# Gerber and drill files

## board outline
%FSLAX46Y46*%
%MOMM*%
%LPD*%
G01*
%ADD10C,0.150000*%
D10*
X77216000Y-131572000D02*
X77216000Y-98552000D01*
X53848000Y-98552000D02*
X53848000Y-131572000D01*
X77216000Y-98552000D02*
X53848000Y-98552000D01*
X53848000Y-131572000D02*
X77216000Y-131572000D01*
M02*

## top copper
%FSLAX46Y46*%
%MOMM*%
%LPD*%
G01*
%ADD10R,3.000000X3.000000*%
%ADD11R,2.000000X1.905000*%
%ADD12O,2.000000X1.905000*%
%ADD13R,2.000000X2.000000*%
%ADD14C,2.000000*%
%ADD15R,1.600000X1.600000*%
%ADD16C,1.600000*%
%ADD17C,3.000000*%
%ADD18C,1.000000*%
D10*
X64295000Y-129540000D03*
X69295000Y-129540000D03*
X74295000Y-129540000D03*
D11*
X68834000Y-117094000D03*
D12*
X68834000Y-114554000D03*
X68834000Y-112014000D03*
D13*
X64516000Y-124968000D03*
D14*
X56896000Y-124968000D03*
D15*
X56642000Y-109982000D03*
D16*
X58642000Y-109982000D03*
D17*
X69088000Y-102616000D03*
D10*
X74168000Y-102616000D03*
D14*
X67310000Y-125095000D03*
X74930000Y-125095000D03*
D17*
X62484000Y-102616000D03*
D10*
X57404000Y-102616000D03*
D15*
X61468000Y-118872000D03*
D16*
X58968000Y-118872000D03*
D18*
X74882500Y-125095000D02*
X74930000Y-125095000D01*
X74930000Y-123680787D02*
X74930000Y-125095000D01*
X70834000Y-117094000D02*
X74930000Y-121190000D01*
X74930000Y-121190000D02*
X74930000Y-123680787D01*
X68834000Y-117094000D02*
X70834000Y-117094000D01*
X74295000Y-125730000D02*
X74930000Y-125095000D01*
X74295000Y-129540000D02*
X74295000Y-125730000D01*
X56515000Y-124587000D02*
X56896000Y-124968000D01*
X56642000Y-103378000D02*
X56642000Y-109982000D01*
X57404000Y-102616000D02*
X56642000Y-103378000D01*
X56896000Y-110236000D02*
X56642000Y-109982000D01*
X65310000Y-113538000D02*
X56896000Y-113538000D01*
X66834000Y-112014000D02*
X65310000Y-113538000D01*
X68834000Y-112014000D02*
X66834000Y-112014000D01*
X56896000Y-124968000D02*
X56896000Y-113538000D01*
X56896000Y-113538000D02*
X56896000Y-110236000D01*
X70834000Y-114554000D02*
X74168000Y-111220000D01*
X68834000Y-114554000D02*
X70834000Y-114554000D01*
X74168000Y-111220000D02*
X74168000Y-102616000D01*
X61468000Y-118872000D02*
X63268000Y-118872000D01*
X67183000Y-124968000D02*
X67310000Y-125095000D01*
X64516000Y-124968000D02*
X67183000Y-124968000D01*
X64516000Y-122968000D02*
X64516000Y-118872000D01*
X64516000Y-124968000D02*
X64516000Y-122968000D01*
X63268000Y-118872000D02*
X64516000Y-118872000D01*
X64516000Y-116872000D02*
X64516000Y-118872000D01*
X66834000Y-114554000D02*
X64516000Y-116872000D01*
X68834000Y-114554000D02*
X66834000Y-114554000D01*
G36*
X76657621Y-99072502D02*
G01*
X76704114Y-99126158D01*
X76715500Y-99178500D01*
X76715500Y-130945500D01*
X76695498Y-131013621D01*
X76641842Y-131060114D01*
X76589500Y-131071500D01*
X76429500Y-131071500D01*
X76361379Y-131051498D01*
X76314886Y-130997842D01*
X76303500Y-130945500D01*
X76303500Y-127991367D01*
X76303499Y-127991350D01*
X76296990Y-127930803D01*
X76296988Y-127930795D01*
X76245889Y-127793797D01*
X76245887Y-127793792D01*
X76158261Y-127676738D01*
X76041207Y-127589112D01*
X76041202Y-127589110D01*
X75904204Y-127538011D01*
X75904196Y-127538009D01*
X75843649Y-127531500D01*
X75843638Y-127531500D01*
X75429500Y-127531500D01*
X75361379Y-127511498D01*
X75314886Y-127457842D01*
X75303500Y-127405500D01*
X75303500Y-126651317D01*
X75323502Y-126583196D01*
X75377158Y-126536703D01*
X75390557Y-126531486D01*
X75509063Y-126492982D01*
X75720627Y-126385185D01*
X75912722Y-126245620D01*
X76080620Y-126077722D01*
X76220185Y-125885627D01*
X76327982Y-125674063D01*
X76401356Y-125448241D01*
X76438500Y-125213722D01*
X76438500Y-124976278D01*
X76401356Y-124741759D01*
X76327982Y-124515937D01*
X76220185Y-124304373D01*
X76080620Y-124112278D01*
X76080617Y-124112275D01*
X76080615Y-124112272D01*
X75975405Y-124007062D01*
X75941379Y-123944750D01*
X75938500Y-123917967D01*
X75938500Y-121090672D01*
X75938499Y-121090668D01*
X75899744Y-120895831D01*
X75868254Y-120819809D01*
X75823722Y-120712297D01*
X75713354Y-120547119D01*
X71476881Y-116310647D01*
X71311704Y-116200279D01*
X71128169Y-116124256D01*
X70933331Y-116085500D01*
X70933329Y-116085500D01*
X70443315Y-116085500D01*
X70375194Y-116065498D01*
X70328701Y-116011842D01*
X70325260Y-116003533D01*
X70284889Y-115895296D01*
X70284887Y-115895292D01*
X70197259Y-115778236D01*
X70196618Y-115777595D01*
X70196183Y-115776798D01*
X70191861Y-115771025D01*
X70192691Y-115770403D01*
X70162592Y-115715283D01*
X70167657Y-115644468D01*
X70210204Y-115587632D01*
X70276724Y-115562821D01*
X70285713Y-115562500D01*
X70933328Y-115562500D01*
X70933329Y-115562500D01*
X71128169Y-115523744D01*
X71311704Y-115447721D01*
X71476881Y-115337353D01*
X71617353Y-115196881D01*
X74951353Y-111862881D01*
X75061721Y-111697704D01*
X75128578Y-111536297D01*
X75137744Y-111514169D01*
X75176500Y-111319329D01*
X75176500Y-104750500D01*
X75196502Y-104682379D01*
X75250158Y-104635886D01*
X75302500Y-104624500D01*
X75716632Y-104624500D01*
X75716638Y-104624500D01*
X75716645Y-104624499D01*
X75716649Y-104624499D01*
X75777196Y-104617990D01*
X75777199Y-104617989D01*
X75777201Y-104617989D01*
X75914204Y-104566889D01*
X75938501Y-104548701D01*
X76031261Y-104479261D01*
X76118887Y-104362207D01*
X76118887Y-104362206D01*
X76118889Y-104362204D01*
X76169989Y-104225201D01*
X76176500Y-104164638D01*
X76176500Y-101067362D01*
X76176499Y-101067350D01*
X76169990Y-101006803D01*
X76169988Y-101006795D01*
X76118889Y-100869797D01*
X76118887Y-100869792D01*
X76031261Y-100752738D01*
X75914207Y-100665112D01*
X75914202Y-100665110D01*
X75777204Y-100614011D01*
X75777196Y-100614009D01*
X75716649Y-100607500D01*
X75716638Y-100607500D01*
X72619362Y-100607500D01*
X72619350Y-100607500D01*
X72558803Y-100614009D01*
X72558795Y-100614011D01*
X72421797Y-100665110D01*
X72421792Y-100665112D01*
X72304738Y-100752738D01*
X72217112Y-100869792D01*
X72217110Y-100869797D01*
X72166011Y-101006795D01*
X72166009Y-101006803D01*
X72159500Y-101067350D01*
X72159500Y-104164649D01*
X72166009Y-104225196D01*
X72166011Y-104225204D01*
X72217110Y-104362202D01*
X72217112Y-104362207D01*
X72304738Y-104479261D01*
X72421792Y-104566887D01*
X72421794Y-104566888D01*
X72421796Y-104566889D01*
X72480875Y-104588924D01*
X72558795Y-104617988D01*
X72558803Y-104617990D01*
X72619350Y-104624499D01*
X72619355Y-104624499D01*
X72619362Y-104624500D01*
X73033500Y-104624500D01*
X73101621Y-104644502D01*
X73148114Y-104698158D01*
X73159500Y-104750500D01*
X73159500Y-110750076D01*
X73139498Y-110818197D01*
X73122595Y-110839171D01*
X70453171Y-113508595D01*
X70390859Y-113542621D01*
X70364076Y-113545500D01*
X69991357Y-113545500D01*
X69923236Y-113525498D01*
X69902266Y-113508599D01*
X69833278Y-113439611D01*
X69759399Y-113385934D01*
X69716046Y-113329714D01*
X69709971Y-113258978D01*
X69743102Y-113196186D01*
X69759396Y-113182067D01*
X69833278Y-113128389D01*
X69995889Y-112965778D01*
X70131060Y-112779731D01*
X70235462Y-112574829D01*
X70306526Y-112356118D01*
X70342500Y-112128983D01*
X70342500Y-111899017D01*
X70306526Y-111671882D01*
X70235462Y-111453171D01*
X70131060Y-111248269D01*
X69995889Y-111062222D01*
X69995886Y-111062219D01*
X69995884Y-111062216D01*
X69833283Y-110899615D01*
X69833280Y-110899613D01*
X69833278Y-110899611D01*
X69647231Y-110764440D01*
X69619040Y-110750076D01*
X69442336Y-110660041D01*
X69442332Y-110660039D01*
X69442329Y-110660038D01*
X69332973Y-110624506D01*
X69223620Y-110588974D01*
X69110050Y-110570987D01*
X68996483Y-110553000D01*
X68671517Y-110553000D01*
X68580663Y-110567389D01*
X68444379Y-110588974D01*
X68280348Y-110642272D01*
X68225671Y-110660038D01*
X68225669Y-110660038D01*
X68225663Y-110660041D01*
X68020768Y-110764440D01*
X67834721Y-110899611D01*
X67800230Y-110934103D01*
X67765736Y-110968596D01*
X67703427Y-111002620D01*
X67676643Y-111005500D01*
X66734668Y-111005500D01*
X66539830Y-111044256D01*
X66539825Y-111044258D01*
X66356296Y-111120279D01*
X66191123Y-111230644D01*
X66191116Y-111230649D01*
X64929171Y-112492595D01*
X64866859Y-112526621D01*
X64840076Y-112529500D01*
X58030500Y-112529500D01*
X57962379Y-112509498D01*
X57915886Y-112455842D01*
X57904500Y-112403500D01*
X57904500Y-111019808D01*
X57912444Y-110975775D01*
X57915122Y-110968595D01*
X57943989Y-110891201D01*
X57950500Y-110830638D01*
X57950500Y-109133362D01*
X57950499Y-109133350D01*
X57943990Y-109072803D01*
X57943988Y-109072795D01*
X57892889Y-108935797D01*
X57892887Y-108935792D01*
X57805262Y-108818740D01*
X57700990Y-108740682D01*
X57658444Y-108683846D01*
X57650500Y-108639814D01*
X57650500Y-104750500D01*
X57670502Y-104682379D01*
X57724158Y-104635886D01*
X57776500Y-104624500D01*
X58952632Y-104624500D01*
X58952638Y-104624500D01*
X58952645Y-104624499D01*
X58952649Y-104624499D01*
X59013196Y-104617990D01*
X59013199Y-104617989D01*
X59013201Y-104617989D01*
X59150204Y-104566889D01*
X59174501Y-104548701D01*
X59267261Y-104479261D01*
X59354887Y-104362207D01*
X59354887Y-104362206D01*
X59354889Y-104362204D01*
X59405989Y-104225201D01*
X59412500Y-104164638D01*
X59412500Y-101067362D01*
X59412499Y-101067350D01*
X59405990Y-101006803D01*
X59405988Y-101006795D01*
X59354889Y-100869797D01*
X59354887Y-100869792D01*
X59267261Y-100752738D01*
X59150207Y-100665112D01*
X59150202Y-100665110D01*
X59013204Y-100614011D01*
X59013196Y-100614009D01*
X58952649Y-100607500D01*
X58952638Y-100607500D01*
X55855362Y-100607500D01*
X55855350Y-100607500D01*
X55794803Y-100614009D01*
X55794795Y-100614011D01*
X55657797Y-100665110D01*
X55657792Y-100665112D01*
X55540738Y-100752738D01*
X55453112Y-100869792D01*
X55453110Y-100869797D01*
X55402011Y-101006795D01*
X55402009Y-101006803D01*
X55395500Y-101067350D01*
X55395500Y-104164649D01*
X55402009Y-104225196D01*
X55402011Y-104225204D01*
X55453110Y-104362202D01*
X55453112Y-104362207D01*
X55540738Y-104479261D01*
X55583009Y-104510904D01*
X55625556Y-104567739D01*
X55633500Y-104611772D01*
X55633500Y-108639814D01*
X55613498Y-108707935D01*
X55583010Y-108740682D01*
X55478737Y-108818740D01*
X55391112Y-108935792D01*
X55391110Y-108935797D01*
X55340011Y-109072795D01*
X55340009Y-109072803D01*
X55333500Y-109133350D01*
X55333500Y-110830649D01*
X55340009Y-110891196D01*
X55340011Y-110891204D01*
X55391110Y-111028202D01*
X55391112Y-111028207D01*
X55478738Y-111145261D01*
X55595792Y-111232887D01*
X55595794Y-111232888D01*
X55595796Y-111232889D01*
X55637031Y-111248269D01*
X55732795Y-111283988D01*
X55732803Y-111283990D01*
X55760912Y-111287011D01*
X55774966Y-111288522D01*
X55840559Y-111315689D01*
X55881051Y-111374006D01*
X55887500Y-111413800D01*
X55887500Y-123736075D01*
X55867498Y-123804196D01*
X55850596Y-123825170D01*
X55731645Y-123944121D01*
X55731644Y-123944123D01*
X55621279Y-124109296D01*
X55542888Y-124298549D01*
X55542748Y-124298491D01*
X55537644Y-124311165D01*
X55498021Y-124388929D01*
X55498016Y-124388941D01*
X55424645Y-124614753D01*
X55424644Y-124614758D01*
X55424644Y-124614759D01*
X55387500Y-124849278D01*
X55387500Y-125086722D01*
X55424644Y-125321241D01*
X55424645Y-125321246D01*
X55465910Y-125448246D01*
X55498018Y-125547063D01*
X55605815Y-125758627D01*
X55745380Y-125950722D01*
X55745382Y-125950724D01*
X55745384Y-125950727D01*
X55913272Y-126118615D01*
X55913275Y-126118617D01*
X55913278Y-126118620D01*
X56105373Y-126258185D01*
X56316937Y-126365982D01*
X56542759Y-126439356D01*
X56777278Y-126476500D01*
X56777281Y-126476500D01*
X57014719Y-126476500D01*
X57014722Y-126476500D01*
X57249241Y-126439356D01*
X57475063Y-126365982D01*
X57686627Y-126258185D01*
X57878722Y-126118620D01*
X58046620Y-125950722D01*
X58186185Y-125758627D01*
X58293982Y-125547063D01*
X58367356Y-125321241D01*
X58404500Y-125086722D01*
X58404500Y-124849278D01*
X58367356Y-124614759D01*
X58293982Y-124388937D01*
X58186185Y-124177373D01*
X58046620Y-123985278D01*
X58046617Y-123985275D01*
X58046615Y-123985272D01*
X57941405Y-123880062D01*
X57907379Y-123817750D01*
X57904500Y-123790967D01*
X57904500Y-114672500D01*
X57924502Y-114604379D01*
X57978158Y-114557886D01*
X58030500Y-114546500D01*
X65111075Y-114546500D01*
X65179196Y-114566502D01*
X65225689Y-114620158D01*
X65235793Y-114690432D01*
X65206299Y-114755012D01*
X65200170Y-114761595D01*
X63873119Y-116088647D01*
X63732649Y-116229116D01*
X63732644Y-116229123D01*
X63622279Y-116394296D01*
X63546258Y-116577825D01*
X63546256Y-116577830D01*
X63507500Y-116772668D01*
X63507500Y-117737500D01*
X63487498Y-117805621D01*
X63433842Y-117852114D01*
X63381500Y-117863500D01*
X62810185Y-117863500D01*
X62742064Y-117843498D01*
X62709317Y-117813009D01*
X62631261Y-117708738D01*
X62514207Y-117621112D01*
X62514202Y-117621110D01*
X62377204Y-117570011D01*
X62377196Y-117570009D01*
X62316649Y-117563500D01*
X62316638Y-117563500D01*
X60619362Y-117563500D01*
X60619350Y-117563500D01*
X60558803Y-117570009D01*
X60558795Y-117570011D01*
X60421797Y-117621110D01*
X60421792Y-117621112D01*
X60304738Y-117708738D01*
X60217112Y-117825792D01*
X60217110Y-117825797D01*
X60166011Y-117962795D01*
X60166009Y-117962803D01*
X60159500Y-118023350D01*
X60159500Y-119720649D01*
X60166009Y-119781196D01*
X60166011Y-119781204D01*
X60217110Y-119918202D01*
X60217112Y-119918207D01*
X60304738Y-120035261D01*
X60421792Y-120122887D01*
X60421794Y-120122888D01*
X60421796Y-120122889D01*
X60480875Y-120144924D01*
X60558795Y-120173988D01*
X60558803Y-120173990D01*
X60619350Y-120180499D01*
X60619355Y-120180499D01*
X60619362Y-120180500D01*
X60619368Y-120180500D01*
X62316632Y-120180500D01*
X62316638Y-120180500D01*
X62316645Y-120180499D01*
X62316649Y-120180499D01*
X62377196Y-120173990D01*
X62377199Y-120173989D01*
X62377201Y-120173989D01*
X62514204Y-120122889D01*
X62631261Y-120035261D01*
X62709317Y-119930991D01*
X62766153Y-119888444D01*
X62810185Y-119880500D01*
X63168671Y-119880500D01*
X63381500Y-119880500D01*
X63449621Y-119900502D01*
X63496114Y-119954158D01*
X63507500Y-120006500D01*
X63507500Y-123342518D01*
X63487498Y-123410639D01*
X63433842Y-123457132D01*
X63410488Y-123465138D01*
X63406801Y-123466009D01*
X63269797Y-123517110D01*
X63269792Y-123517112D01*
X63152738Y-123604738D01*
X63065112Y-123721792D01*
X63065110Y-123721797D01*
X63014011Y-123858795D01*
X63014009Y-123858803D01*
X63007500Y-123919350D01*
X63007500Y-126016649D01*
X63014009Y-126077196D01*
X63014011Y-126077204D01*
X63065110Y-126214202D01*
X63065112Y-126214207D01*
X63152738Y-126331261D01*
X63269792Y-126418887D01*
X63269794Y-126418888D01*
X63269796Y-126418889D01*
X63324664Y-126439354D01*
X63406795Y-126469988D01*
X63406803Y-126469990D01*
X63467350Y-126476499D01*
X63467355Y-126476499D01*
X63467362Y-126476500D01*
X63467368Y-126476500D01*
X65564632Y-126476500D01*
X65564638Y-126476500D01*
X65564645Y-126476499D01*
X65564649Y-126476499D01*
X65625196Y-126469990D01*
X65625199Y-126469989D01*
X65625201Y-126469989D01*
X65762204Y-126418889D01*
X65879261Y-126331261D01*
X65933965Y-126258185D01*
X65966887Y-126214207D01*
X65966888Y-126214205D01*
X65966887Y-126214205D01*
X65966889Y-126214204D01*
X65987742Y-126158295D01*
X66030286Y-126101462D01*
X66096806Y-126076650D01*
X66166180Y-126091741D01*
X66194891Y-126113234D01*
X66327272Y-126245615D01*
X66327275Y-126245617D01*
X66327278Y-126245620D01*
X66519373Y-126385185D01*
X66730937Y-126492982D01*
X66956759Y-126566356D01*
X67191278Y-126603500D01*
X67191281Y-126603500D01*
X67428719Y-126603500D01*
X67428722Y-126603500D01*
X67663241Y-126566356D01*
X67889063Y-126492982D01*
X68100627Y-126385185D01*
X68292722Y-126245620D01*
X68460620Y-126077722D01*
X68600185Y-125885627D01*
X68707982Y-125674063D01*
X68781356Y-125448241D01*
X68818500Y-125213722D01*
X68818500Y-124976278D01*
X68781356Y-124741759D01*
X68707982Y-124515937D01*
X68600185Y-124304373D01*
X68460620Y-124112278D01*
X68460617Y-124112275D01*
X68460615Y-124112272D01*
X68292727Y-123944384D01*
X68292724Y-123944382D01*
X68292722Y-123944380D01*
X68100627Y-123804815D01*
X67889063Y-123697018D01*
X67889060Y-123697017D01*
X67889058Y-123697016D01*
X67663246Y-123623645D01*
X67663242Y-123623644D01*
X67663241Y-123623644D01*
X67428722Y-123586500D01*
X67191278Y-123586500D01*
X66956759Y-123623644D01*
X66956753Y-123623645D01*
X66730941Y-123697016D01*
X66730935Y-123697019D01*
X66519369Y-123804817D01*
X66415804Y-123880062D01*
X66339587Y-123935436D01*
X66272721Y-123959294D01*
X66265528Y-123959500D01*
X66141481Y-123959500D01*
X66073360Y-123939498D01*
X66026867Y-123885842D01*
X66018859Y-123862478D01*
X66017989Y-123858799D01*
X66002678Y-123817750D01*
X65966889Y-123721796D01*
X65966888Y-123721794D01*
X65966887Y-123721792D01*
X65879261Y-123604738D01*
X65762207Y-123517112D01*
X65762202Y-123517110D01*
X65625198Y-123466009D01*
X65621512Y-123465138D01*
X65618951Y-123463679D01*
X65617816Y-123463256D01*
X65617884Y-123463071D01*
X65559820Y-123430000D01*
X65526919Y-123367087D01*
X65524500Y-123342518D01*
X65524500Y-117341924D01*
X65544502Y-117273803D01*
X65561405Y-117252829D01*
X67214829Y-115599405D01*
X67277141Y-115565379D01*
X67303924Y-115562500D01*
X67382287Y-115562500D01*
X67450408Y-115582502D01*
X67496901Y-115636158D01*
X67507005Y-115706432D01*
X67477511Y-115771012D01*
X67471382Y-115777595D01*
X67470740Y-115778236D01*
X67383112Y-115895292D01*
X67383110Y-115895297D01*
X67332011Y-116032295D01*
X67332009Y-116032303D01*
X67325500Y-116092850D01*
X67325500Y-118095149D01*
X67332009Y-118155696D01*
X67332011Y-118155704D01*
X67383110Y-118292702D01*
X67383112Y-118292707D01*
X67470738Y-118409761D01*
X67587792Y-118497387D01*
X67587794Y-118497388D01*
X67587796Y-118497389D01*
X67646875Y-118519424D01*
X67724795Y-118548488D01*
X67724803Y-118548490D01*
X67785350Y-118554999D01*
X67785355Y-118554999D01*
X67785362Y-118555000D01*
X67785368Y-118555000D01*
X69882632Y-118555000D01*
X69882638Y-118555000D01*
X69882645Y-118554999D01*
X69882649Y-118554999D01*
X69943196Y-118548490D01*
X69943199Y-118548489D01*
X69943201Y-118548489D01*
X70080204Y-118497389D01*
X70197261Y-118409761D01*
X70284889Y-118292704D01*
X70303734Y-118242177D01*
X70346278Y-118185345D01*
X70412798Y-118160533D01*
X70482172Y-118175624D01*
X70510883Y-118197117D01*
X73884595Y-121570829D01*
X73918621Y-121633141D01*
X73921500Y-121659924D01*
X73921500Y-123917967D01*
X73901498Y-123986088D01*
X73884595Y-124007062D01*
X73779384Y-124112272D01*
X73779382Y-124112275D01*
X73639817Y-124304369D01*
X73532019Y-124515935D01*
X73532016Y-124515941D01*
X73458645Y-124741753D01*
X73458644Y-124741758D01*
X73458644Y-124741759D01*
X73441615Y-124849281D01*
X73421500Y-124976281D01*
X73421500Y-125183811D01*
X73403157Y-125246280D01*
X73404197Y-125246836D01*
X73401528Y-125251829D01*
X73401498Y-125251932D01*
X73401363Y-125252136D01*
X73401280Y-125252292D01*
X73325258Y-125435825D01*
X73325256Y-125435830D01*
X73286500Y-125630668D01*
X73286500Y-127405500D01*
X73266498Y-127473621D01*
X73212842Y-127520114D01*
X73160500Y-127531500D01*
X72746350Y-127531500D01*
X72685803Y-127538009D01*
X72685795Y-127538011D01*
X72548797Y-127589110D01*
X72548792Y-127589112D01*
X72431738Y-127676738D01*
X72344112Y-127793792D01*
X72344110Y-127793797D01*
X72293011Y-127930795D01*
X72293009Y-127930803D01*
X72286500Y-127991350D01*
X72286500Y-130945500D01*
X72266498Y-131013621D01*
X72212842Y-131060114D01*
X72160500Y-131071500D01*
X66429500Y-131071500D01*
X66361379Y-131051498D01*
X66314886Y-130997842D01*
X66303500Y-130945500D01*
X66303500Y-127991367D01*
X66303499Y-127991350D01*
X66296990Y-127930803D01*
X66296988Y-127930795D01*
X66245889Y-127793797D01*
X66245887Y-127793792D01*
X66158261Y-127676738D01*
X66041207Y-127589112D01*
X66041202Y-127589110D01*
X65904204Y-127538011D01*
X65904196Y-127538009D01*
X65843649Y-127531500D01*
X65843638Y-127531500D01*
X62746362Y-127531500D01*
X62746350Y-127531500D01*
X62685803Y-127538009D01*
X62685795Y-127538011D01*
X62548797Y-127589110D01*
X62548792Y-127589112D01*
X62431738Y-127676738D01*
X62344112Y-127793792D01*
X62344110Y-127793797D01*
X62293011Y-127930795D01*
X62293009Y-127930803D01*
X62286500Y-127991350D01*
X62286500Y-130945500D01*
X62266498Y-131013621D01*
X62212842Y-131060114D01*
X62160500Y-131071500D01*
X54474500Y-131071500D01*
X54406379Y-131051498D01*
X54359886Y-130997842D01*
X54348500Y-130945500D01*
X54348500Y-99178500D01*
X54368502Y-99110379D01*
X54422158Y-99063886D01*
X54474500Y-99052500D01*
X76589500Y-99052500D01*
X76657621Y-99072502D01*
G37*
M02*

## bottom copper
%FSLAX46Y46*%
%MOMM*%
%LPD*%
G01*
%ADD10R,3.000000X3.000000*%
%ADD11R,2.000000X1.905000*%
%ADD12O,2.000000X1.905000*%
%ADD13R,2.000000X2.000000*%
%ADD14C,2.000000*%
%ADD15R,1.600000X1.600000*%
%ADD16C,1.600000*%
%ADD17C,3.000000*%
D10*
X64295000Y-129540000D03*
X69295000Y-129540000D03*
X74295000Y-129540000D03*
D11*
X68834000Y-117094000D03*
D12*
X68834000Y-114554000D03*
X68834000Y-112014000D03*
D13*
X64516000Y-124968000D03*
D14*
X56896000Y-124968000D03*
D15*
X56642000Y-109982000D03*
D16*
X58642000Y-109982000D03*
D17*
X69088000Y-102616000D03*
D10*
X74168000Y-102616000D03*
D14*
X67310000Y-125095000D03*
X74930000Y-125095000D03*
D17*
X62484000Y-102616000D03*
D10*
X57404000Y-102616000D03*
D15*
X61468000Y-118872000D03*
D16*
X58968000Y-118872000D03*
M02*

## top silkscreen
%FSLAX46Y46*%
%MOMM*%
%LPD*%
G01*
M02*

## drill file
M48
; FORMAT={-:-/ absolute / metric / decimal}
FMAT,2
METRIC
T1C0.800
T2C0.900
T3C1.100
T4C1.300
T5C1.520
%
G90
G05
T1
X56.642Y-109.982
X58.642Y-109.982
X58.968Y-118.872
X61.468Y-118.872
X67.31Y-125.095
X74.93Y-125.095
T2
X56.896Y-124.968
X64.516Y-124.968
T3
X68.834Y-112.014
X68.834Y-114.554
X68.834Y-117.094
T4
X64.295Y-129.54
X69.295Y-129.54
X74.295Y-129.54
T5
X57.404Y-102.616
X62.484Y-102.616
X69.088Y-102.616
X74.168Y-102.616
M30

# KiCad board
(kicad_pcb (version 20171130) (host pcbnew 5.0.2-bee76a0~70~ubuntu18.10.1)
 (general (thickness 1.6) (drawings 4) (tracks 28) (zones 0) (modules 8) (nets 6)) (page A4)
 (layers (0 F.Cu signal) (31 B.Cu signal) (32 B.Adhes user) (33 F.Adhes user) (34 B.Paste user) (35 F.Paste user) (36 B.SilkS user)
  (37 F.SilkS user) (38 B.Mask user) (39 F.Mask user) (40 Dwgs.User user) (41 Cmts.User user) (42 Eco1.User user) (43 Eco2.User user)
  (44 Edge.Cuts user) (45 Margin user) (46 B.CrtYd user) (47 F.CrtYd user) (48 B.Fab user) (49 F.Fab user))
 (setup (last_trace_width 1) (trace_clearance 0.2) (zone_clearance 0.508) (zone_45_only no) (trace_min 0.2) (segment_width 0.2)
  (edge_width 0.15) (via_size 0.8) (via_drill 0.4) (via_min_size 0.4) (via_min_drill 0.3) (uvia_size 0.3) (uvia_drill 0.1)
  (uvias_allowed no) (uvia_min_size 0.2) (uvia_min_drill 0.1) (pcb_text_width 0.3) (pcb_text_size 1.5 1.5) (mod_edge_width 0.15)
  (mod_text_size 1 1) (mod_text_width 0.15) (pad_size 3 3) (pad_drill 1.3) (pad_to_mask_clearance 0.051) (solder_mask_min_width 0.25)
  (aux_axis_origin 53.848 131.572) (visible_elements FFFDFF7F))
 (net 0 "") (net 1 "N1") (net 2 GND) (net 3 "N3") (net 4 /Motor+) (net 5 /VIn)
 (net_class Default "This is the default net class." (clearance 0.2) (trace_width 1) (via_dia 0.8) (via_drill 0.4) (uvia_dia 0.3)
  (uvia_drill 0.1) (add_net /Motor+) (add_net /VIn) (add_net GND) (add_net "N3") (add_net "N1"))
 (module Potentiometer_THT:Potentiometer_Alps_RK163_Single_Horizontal (layer B.Cu) (at 74.295 129.54 270)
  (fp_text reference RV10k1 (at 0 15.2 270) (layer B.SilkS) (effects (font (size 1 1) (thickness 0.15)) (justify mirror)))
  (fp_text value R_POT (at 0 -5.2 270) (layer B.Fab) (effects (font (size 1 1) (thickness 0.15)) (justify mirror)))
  (pad 3 thru_hole rect (at 0 10 270) (size 3 3) (drill 1.3) (layers *.Cu *.Mask) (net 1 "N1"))
  (pad 2 thru_hole rect (at 0 5 270) (size 3 3) (drill 1.3) (layers *.Cu *.Mask) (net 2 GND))
  (pad 1 thru_hole rect (at 0 0 270) (size 3 3) (drill 1.3) (layers *.Cu *.Mask) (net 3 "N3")))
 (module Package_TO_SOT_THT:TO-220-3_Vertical (layer B.Cu) (at 68.834 117.094 90)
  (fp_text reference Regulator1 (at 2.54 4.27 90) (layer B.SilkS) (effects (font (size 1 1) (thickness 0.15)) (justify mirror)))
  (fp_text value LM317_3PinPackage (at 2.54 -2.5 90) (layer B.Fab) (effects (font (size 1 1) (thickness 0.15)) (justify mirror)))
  (pad 1 thru_hole rect (at 0 0 90) (size 1.905 2) (drill 1.1) (layers *.Cu *.Mask) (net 3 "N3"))
  (pad 2 thru_hole oval (at 2.54 0 90) (size 1.905 2) (drill 1.1) (layers *.Cu *.Mask) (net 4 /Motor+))
  (pad 3 thru_hole oval (at 5.08 0 90) (size 1.905 2) (drill 1.1) (layers *.Cu *.Mask) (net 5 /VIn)))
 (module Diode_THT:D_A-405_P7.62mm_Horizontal (layer B.Cu) (at 64.516 124.968 180)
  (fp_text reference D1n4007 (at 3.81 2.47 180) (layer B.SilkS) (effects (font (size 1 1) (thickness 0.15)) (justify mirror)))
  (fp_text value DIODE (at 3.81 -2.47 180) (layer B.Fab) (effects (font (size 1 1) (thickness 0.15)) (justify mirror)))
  (pad 1 thru_hole rect (at 0 0 180) (size 2 2) (drill 0.9) (layers *.Cu *.Mask) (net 4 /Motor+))
  (pad 2 thru_hole circle (at 7.62 0 180) (size 2 2) (drill 0.9) (layers *.Cu *.Mask) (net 5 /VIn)))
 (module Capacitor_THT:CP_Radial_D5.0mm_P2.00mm (layer B.Cu) (at 56.642 109.982)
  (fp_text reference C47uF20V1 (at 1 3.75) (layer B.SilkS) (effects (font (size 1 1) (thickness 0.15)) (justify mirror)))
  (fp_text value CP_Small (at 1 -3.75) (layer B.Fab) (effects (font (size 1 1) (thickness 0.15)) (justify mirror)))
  (pad 1 thru_hole rect (at 0 0) (size 1.6 1.6) (drill 0.8) (layers *.Cu *.Mask) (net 5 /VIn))
  (pad 2 thru_hole circle (at 2 0) (size 1.6 1.6) (drill 0.8) (layers *.Cu *.Mask) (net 2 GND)))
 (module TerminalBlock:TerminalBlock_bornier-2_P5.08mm (layer B.Cu) (at 74.168 102.616 180)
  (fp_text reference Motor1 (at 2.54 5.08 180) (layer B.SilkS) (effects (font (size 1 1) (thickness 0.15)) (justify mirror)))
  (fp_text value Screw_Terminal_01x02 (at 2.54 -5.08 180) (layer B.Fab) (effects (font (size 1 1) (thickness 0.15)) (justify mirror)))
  (pad 2 thru_hole circle (at 5.08 0 180) (size 3 3) (drill 1.52) (layers *.Cu *.Mask) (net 2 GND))
  (pad 1 thru_hole rect (at 0 0 180) (size 3 3) (drill 1.52) (layers *.Cu *.Mask) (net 4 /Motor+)))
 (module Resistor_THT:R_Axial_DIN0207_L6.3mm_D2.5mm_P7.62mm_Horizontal (layer B.Cu) (at 67.31 125.095)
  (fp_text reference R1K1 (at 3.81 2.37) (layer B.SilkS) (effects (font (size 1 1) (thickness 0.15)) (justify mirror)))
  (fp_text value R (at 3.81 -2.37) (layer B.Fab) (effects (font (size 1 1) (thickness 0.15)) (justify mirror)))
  (pad 1 thru_hole circle (at 0 0) (size 2 2) (drill 0.8) (layers *.Cu *.Mask) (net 4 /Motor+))
  (pad 2 thru_hole circle (at 7.62 0) (size 2 2) (drill 0.8) (layers *.Cu *.Mask) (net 3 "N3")))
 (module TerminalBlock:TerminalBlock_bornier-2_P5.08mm (layer B.Cu) (at 62.484 102.616 180)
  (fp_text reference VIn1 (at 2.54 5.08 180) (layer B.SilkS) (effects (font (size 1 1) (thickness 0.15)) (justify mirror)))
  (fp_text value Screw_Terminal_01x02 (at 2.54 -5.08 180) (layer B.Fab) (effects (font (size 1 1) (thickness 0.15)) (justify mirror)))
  (pad 1 thru_hole circle (at 0 0 180) (size 3 3) (drill 1.52) (layers *.Cu *.Mask) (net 2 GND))
  (pad 2 thru_hole rect (at 5.08 0 180) (size 3 3) (drill 1.52) (layers *.Cu *.Mask) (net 5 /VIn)))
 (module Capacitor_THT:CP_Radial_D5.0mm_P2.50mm (layer B.Cu) (at 61.468 118.872 180)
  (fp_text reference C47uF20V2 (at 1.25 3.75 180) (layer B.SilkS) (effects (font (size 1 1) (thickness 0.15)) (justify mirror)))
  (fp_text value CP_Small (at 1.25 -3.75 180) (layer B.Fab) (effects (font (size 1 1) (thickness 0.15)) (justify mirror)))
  (pad 1 thru_hole rect (at 0 0 180) (size 1.6 1.6) (drill 0.8) (layers *.Cu *.Mask) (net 4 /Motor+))
  (pad 2 thru_hole circle (at 2.5 0 180) (size 1.6 1.6) (drill 0.8) (layers *.Cu *.Mask) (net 2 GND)))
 (gr_line (start 77.216 131.572) (end 77.216 98.552) (layer Edge.Cuts) (width 0.15))
 (gr_line (start 53.848 98.552) (end 53.848 131.572) (layer Edge.Cuts) (width 0.15))
 (gr_line (start 77.216 98.552) (end 53.848 98.552) (layer Edge.Cuts) (width 0.15))
 (gr_line (start 53.848 131.572) (end 77.216 131.572) (layer Edge.Cuts) (width 0.15))
 (segment (start 74.8825 125.095) (end 74.93 125.095) (width 1) (layer F.Cu) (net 3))
 (segment (start 74.93 123.680787) (end 74.93 125.095) (width 1) (layer F.Cu) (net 3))
 (segment (start 70.834 117.094) (end 74.93 121.19) (width 1) (layer F.Cu) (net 3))
 (segment (start 74.93 121.19) (end 74.93 123.680787) (width 1) (layer F.Cu) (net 3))
 (segment (start 68.834 117.094) (end 70.834 117.094) (width 1) (layer F.Cu) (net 3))
 (segment (start 74.295 125.73) (end 74.93 125.095) (width 1) (layer F.Cu) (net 3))
 (segment (start 74.295 129.54) (end 74.295 125.73) (width 1) (layer F.Cu) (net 3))
 (segment (start 56.515 124.587) (end 56.896 124.968) (width 1) (layer F.Cu) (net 5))
 (segment (start 56.642 103.378) (end 56.642 109.982) (width 1) (layer F.Cu) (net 5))
 (segment (start 57.404 102.616) (end 56.642 103.378) (width 1) (layer F.Cu) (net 5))
 (segment (start 56.896 110.236) (end 56.642 109.982) (width 1) (layer F.Cu) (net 5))
 (segment (start 65.31 113.538) (end 56.896 113.538) (width 1) (layer F.Cu) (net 5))
 (segment (start 66.834 112.014) (end 65.31 113.538) (width 1) (layer F.Cu) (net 5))
 (segment (start 68.834 112.014) (end 66.834 112.014) (width 1) (layer F.Cu) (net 5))
 (segment (start 56.896 124.968) (end 56.896 113.538) (width 1) (layer F.Cu) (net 5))
 (segment (start 56.896 113.538) (end 56.896 110.236) (width 1) (layer F.Cu) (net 5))
 (segment (start 70.834 114.554) (end 74.168 111.22) (width 1) (layer F.Cu) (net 4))
 (segment (start 68.834 114.554) (end 70.834 114.554) (width 1) (layer F.Cu) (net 4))
 (segment (start 74.168 111.22) (end 74.168 102.616) (width 1) (layer F.Cu) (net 4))
 (segment (start 61.468 118.872) (end 63.268 118.872) (width 1) (layer F.Cu) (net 4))
 (segment (start 67.183 124.968) (end 67.31 125.095) (width 1) (layer F.Cu) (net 4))
 (segment (start 64.516 124.968) (end 67.183 124.968) (width 1) (layer F.Cu) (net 4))
 (segment (start 64.516 122.968) (end 64.516 118.872) (width 1) (layer F.Cu) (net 4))
 (segment (start 64.516 124.968) (end 64.516 122.968) (width 1) (layer F.Cu) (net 4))
 (segment (start 63.268 118.872) (end 64.516 118.872) (width 1) (layer F.Cu) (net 4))
 (segment (start 64.516 116.872) (end 64.516 118.872) (width 1) (layer F.Cu) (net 4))
 (segment (start 66.834 114.554) (end 64.516 116.872) (width 1) (layer F.Cu) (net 4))
 (segment (start 68.834 114.554) (end 66.834 114.554) (width 1) (layer F.Cu) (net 4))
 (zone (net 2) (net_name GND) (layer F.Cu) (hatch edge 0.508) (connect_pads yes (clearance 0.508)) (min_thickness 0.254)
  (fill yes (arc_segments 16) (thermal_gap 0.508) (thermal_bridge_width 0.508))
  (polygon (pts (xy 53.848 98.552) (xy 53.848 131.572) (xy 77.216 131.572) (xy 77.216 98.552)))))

